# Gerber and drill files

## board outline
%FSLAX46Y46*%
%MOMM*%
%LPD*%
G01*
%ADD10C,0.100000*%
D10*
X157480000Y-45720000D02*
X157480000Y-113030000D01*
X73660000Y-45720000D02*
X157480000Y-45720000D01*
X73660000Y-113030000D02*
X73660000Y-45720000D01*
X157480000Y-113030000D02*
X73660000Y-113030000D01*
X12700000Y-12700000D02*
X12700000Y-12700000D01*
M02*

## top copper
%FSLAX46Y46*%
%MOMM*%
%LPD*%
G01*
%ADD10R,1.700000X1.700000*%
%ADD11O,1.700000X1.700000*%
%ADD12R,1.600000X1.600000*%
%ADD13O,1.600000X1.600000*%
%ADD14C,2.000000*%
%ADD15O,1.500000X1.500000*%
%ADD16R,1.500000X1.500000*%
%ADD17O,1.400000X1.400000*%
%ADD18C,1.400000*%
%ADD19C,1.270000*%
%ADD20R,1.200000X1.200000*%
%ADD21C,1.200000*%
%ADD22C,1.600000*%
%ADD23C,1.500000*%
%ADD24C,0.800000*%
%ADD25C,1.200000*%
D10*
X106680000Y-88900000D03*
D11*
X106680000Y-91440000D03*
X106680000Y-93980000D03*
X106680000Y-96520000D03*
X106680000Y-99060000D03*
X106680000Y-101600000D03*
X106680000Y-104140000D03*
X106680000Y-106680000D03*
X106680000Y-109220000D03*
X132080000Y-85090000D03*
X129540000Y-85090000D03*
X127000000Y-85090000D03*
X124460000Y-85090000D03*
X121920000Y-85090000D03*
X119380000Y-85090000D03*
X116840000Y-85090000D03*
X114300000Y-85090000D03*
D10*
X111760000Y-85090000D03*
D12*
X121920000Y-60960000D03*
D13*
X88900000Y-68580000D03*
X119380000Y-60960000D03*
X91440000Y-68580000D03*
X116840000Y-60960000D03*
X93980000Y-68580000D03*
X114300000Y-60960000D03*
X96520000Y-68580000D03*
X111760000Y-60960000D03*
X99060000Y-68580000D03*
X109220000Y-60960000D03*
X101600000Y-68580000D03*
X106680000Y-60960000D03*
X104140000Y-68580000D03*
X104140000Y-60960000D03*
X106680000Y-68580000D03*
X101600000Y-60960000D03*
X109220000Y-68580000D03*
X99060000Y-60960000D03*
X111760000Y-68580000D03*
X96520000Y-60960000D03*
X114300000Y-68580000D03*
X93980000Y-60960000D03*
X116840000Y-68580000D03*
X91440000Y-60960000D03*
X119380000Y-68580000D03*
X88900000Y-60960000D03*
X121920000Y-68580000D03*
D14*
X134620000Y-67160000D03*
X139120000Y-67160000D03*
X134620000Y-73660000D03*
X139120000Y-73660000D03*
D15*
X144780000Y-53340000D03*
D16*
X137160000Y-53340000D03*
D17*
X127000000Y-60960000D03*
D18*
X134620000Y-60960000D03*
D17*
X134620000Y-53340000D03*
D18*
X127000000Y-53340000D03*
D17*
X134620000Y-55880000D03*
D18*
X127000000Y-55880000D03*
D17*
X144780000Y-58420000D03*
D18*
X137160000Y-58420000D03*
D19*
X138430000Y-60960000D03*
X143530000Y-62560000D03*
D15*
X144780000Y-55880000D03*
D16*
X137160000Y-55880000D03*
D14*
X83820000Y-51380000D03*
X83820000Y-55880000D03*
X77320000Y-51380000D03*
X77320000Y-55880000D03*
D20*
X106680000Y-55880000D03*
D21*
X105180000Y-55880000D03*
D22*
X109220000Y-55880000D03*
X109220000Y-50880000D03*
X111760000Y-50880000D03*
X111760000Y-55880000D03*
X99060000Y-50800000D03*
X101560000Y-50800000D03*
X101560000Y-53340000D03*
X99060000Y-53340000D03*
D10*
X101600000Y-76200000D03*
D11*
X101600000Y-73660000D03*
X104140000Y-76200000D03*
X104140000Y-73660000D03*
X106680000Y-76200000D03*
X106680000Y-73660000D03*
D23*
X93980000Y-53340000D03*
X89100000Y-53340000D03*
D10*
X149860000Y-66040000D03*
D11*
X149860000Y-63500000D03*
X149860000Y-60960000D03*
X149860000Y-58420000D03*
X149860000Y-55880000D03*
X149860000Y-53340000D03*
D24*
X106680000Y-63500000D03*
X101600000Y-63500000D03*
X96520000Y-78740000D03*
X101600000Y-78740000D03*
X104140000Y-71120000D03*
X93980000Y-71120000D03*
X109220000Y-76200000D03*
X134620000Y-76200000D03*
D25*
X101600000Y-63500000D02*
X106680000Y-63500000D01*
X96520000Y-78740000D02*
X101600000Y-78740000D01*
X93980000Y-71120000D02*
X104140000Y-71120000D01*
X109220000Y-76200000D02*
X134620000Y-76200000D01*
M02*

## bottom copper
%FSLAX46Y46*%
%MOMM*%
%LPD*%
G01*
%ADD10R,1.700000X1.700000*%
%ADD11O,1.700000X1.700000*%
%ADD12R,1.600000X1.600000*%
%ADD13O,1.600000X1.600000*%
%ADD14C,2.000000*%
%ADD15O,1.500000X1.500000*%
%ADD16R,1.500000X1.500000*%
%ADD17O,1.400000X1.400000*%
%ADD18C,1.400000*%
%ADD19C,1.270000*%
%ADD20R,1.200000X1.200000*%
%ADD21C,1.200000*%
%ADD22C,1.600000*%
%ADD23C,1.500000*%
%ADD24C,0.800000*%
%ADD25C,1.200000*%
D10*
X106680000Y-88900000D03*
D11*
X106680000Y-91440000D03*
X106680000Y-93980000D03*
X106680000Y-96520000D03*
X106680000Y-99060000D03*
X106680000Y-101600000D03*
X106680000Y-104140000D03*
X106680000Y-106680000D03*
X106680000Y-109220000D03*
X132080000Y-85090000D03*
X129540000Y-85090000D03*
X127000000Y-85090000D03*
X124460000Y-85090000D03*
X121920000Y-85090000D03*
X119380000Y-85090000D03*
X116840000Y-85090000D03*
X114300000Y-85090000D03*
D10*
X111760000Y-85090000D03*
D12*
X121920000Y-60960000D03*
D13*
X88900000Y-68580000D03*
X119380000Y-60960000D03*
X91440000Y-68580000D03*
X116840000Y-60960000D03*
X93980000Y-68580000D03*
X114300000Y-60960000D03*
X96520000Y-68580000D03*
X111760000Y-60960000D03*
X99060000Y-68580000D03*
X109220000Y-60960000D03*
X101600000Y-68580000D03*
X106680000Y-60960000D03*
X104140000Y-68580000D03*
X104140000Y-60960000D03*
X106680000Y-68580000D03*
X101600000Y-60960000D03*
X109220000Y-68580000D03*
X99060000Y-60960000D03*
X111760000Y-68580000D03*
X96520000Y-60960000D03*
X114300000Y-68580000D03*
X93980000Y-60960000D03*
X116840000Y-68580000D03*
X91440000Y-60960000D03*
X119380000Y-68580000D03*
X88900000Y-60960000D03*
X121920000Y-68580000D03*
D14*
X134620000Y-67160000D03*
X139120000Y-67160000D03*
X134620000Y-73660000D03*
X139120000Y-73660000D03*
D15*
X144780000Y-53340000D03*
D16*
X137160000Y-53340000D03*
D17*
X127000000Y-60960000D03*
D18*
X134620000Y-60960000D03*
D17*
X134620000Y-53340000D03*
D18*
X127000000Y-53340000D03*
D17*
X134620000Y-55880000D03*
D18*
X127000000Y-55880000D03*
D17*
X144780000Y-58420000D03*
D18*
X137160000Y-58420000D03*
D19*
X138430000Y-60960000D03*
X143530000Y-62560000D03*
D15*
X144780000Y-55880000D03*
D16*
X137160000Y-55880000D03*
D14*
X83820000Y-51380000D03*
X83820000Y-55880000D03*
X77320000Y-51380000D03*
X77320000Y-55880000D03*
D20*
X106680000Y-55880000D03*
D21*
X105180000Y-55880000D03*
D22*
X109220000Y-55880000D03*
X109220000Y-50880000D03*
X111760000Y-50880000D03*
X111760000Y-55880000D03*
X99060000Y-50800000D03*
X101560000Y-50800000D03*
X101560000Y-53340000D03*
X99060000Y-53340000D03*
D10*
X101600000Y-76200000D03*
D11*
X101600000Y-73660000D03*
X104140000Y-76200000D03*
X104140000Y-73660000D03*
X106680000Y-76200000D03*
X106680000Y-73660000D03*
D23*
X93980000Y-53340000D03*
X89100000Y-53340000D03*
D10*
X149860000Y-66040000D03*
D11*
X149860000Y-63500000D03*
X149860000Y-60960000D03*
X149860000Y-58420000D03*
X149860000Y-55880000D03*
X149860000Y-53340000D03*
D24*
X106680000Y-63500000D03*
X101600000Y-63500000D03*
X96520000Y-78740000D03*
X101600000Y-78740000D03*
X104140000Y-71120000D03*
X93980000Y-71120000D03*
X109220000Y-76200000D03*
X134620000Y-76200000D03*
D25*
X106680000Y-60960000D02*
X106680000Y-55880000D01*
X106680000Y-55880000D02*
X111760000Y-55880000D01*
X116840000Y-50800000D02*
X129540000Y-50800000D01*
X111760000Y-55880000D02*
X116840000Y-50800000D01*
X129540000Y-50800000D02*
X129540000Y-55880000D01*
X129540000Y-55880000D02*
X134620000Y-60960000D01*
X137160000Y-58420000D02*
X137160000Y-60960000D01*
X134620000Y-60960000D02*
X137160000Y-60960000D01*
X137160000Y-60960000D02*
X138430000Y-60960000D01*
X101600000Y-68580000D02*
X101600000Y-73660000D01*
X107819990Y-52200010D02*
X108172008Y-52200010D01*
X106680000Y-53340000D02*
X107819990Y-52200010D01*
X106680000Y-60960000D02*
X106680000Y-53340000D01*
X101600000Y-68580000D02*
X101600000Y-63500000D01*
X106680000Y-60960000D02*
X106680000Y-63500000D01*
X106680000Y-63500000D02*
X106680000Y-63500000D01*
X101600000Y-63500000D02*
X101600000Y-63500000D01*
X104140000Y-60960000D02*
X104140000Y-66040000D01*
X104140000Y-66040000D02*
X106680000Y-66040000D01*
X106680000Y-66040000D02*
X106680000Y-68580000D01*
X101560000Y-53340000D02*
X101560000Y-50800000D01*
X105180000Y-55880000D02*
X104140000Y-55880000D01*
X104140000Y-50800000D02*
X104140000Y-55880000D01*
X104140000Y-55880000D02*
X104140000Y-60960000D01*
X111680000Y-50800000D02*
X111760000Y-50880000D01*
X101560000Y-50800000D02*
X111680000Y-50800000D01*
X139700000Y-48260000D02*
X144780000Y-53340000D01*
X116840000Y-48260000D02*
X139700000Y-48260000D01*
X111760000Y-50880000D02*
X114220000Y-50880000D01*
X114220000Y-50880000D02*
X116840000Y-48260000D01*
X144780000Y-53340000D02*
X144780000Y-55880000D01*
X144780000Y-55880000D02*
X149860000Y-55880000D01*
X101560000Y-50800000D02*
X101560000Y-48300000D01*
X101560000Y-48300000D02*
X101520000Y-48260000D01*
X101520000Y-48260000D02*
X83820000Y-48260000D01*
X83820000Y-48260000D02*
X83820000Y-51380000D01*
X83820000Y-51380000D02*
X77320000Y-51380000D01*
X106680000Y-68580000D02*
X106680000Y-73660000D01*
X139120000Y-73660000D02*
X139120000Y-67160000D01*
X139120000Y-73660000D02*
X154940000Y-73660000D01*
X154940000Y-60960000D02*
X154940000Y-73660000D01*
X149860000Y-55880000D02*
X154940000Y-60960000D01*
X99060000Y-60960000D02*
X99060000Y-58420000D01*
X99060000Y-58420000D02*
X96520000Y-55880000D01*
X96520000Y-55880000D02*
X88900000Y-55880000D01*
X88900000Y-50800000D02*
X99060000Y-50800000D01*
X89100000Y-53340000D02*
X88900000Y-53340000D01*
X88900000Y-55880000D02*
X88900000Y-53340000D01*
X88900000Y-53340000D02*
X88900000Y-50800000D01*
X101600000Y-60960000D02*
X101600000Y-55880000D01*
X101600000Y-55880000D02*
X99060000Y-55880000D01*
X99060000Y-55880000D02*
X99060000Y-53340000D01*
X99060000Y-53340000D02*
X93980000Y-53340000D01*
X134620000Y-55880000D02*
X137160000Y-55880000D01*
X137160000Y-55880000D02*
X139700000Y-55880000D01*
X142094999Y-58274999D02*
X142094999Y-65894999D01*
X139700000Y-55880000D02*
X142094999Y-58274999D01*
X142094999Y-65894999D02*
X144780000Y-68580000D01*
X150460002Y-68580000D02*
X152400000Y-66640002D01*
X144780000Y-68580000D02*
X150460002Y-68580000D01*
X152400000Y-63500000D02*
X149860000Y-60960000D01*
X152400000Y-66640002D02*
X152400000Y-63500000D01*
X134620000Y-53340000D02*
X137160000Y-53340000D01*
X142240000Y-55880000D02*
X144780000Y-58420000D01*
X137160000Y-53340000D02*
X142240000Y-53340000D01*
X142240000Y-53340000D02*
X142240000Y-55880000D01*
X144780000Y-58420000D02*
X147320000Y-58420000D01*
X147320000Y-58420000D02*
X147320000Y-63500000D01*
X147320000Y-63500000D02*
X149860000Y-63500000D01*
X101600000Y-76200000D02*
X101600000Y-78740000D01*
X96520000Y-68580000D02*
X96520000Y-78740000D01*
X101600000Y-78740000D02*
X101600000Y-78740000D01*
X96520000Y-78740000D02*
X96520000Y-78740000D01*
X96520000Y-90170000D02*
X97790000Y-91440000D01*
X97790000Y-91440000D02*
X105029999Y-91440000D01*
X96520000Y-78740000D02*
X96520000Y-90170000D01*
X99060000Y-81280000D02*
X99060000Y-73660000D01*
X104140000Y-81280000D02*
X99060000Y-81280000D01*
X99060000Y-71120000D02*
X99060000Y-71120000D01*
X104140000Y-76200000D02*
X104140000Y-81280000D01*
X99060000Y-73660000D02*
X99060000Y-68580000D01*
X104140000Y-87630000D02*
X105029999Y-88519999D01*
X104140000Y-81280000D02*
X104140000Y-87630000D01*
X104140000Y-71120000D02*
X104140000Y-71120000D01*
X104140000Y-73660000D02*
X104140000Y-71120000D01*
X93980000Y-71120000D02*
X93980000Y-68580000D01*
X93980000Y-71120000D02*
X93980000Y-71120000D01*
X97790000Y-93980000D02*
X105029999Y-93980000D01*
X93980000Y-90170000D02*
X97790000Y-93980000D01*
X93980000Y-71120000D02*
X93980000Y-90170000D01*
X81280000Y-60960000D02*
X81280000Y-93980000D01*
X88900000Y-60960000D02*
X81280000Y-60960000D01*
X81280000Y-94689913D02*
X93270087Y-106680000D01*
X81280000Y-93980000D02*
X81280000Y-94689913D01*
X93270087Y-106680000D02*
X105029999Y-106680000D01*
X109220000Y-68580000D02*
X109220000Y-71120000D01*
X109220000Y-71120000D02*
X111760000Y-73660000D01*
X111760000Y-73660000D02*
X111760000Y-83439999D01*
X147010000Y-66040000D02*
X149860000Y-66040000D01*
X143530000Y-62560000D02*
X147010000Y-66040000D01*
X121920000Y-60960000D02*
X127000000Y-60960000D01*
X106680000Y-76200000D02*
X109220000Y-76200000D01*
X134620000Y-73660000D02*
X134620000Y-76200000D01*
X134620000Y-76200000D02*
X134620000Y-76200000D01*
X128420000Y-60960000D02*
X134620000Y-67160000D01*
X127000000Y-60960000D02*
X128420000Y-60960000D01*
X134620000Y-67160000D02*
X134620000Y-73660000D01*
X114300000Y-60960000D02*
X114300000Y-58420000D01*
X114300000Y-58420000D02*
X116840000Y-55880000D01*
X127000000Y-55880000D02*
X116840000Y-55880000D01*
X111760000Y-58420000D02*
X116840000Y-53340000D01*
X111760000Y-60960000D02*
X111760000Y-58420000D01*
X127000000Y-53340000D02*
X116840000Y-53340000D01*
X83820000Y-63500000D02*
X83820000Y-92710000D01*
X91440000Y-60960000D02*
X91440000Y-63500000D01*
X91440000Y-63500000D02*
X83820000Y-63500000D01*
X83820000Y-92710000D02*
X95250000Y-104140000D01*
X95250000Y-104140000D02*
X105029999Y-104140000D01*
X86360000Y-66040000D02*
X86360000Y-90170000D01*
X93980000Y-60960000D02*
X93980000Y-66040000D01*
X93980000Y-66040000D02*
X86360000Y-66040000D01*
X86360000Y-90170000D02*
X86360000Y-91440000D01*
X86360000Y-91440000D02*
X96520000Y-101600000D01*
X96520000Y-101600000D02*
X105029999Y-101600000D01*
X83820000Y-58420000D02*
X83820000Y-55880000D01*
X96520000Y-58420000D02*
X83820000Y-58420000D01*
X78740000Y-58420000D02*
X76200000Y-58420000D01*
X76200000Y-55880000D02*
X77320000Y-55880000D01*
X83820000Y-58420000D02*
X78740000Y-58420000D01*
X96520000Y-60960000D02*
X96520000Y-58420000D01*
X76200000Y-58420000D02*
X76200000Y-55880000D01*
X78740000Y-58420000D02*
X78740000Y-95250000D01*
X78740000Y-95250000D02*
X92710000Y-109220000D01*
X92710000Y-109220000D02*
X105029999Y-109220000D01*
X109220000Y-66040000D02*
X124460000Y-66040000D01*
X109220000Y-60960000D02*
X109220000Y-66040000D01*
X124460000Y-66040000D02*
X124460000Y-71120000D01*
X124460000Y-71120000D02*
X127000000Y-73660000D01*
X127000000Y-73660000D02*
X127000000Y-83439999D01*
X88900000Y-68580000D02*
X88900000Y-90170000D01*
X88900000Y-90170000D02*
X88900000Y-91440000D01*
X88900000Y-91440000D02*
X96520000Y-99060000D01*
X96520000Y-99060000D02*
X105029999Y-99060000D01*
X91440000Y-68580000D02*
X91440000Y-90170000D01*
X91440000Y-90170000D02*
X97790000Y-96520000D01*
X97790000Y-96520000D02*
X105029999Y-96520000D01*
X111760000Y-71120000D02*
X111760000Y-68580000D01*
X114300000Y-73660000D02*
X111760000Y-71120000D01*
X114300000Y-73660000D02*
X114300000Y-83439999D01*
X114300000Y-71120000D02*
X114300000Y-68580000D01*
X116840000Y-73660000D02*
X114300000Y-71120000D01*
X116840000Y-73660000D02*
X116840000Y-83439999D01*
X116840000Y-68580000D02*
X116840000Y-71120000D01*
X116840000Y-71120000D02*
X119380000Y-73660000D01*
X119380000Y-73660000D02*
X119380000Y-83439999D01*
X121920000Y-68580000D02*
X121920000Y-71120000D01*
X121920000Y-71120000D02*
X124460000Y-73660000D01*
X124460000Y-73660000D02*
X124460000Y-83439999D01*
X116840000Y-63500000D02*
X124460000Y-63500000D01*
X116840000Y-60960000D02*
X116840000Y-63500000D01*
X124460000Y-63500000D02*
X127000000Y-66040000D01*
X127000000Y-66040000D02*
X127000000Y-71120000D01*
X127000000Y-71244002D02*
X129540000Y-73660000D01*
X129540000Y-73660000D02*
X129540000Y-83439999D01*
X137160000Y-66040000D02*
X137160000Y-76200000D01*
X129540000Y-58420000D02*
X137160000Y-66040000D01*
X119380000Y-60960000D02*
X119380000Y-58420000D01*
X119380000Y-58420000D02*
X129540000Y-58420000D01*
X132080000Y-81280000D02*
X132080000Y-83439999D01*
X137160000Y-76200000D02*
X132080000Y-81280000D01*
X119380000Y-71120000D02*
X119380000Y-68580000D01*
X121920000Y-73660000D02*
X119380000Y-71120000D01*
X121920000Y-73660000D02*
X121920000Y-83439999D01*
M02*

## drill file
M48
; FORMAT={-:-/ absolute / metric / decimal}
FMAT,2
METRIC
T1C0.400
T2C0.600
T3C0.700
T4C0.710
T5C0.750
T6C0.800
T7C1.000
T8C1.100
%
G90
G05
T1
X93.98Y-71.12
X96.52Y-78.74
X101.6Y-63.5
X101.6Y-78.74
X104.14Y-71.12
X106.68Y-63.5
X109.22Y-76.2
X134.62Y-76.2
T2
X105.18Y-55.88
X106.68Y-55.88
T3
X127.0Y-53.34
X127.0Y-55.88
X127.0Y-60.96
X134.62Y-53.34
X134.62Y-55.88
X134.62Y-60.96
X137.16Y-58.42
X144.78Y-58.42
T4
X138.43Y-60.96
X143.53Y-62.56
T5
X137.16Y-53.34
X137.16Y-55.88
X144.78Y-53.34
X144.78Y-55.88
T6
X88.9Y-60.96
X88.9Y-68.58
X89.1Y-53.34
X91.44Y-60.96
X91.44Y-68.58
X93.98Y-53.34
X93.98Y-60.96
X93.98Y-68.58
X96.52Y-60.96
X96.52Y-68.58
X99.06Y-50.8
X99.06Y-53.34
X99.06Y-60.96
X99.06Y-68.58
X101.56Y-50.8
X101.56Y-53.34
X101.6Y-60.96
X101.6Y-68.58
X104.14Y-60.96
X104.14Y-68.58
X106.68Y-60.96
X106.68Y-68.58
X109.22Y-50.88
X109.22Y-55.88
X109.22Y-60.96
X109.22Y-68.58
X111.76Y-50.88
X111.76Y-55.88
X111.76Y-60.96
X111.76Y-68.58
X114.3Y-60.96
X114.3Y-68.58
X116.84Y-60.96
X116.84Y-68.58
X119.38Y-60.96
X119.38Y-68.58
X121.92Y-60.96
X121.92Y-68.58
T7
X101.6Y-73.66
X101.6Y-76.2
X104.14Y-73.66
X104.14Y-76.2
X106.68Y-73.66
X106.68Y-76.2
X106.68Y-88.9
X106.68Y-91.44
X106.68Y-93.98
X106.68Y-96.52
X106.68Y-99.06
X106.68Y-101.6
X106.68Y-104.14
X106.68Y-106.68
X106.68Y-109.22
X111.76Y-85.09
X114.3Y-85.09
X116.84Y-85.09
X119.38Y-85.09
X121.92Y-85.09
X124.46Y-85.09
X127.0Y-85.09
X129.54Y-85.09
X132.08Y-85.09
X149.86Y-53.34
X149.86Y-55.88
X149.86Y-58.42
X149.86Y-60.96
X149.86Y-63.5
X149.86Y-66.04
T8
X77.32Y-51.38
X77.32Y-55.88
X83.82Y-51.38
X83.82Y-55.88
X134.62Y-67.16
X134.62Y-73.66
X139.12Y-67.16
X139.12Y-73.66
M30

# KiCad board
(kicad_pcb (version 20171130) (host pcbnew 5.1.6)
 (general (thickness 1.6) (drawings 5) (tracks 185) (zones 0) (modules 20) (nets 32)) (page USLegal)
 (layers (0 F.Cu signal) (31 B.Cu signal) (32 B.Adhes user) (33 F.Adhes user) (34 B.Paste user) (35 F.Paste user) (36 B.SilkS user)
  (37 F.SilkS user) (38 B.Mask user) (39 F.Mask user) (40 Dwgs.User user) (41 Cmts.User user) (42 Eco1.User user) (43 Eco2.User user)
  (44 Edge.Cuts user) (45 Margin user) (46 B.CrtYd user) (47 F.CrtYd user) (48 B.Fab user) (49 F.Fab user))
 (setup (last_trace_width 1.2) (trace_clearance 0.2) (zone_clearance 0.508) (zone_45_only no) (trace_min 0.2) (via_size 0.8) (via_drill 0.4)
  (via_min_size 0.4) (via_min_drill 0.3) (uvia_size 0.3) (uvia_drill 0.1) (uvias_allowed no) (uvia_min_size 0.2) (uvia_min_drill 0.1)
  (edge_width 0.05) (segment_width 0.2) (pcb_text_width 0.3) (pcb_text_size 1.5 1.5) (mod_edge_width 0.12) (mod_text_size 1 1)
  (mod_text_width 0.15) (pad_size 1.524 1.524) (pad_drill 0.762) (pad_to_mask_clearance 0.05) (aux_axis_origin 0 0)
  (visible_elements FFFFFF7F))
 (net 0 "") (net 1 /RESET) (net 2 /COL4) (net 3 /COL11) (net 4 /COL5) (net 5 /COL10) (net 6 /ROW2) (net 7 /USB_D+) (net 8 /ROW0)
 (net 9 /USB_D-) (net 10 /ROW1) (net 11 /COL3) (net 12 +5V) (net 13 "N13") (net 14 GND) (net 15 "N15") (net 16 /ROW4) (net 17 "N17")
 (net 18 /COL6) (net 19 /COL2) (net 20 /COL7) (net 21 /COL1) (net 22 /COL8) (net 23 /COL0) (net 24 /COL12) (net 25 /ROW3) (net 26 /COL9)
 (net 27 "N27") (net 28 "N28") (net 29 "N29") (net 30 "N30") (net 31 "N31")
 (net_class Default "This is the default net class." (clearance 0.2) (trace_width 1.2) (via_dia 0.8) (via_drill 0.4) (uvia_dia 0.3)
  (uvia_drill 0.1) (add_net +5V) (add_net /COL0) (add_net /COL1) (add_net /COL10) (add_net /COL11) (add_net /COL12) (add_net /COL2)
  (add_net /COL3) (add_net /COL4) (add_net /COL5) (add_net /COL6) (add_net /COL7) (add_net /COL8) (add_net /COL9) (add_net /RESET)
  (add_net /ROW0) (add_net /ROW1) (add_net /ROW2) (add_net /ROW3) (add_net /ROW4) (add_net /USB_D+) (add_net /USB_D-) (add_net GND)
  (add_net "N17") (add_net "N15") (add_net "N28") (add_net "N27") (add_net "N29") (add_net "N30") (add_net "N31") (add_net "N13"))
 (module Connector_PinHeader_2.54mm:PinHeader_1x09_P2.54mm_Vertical (layer F.Cu) (at 106.68 88.9)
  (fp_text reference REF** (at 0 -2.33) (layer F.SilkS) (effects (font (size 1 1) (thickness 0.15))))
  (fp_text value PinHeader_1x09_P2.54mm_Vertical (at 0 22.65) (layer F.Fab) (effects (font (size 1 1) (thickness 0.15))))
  (pad 1 thru_hole rect (at 0 0) (size 1.7 1.7) (drill 1) (layers *.Cu *.Mask))
  (pad 2 thru_hole oval (at 0 2.54) (size 1.7 1.7) (drill 1) (layers *.Cu *.Mask))
  (pad 3 thru_hole oval (at 0 5.08) (size 1.7 1.7) (drill 1) (layers *.Cu *.Mask))
  (pad 4 thru_hole oval (at 0 7.62) (size 1.7 1.7) (drill 1) (layers *.Cu *.Mask))
  (pad 5 thru_hole oval (at 0 10.16) (size 1.7 1.7) (drill 1) (layers *.Cu *.Mask))
  (pad 6 thru_hole oval (at 0 12.7) (size 1.7 1.7) (drill 1) (layers *.Cu *.Mask))
  (pad 7 thru_hole oval (at 0 15.24) (size 1.7 1.7) (drill 1) (layers *.Cu *.Mask))
  (pad 8 thru_hole oval (at 0 17.78) (size 1.7 1.7) (drill 1) (layers *.Cu *.Mask))
  (pad 9 thru_hole oval (at 0 20.32) (size 1.7 1.7) (drill 1) (layers *.Cu *.Mask)))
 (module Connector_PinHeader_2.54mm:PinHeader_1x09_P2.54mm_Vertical (layer F.Cu) (at 111.76 85.09 90)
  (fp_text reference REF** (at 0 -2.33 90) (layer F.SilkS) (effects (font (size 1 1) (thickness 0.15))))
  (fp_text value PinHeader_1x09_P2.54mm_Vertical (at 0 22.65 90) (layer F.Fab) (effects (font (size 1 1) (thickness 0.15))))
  (pad 9 thru_hole oval (at 0 20.32 90) (size 1.7 1.7) (drill 1) (layers *.Cu *.Mask))
  (pad 8 thru_hole oval (at 0 17.78 90) (size 1.7 1.7) (drill 1) (layers *.Cu *.Mask))
  (pad 7 thru_hole oval (at 0 15.24 90) (size 1.7 1.7) (drill 1) (layers *.Cu *.Mask))
  (pad 6 thru_hole oval (at 0 12.7 90) (size 1.7 1.7) (drill 1) (layers *.Cu *.Mask))
  (pad 5 thru_hole oval (at 0 10.16 90) (size 1.7 1.7) (drill 1) (layers *.Cu *.Mask))
  (pad 4 thru_hole oval (at 0 7.62 90) (size 1.7 1.7) (drill 1) (layers *.Cu *.Mask))
  (pad 3 thru_hole oval (at 0 5.08 90) (size 1.7 1.7) (drill 1) (layers *.Cu *.Mask))
  (pad 2 thru_hole oval (at 0 2.54 90) (size 1.7 1.7) (drill 1) (layers *.Cu *.Mask))
  (pad 1 thru_hole rect (at 0 0 90) (size 1.7 1.7) (drill 1) (layers *.Cu *.Mask)))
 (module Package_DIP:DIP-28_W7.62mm (layer F.Cu) (at 121.92 60.96 270)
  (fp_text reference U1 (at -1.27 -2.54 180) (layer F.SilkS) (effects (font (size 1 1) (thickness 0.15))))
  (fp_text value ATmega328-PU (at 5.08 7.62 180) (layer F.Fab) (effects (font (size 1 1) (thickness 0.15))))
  (pad 1 thru_hole rect (at 0 0 270) (size 1.6 1.6) (drill 0.8) (layers *.Cu *.Mask) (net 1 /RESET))
  (pad 15 thru_hole oval (at 7.62 33.02 270) (size 1.6 1.6) (drill 0.8) (layers *.Cu *.Mask) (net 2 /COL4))
  (pad 2 thru_hole oval (at 0 2.54 270) (size 1.6 1.6) (drill 0.8) (layers *.Cu *.Mask) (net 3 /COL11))
  (pad 16 thru_hole oval (at 7.62 30.48 270) (size 1.6 1.6) (drill 0.8) (layers *.Cu *.Mask) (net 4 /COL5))
  (pad 3 thru_hole oval (at 0 5.08 270) (size 1.6 1.6) (drill 0.8) (layers *.Cu *.Mask) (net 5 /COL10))
  (pad 17 thru_hole oval (at 7.62 27.94 270) (size 1.6 1.6) (drill 0.8) (layers *.Cu *.Mask) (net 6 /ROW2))
  (pad 4 thru_hole oval (at 0 7.62 270) (size 1.6 1.6) (drill 0.8) (layers *.Cu *.Mask) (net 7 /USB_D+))
  (pad 18 thru_hole oval (at 7.62 25.4 270) (size 1.6 1.6) (drill 0.8) (layers *.Cu *.Mask) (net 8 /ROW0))
  (pad 5 thru_hole oval (at 0 10.16 270) (size 1.6 1.6) (drill 0.8) (layers *.Cu *.Mask) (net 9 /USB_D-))
  (pad 19 thru_hole oval (at 7.62 22.86 270) (size 1.6 1.6) (drill 0.8) (layers *.Cu *.Mask) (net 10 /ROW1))
  (pad 6 thru_hole oval (at 0 12.7 270) (size 1.6 1.6) (drill 0.8) (layers *.Cu *.Mask) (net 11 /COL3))
  (pad 20 thru_hole oval (at 7.62 20.32 270) (size 1.6 1.6) (drill 0.8) (layers *.Cu *.Mask) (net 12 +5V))
  (pad 7 thru_hole oval (at 0 15.24 270) (size 1.6 1.6) (drill 0.8) (layers *.Cu *.Mask) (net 12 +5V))
  (pad 21 thru_hole oval (at 7.62 17.78 270) (size 1.6 1.6) (drill 0.8) (layers *.Cu *.Mask) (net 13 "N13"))
  (pad 8 thru_hole oval (at 0 17.78 270) (size 1.6 1.6) (drill 0.8) (layers *.Cu *.Mask) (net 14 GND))
  (pad 22 thru_hole oval (at 7.62 15.24 270) (size 1.6 1.6) (drill 0.8) (layers *.Cu *.Mask) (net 14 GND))
  (pad 9 thru_hole oval (at 0 20.32 270) (size 1.6 1.6) (drill 0.8) (layers *.Cu *.Mask) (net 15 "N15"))
  (pad 23 thru_hole oval (at 7.62 12.7 270) (size 1.6 1.6) (drill 0.8) (layers *.Cu *.Mask) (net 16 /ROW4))
  (pad 10 thru_hole oval (at 0 22.86 270) (size 1.6 1.6) (drill 0.8) (layers *.Cu *.Mask) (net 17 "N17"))
  (pad 24 thru_hole oval (at 7.62 10.16 270) (size 1.6 1.6) (drill 0.8) (layers *.Cu *.Mask) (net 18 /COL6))
  (pad 11 thru_hole oval (at 0 25.4 270) (size 1.6 1.6) (drill 0.8) (layers *.Cu *.Mask) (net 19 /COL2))
  (pad 25 thru_hole oval (at 7.62 7.62 270) (size 1.6 1.6) (drill 0.8) (layers *.Cu *.Mask) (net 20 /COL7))
  (pad 12 thru_hole oval (at 0 27.94 270) (size 1.6 1.6) (drill 0.8) (layers *.Cu *.Mask) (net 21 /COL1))
  (pad 26 thru_hole oval (at 7.62 5.08 270) (size 1.6 1.6) (drill 0.8) (layers *.Cu *.Mask) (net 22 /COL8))
  (pad 13 thru_hole oval (at 0 30.48 270) (size 1.6 1.6) (drill 0.8) (layers *.Cu *.Mask) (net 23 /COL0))
  (pad 27 thru_hole oval (at 7.62 2.54 270) (size 1.6 1.6) (drill 0.8) (layers *.Cu *.Mask) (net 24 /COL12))
  (pad 14 thru_hole oval (at 0 33.02 270) (size 1.6 1.6) (drill 0.8) (layers *.Cu *.Mask) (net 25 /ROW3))
  (pad 28 thru_hole oval (at 7.62 0 270) (size 1.6 1.6) (drill 0.8) (layers *.Cu *.Mask) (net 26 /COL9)))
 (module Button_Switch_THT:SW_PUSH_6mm (layer F.Cu) (at 134.62 73.66 90)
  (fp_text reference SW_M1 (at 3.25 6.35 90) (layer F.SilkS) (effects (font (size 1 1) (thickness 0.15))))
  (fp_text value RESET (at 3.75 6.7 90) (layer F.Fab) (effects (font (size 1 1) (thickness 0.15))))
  (pad 1 thru_hole circle (at 6.5 0 180) (size 2 2) (drill 1.1) (layers *.Cu *.Mask) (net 1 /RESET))
  (pad 2 thru_hole circle (at 6.5 4.5 180) (size 2 2) (drill 1.1) (layers *.Cu *.Mask) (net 14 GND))
  (pad 1 thru_hole circle (at 0 0 180) (size 2 2) (drill 1.1) (layers *.Cu *.Mask) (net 1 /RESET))
  (pad 2 thru_hole circle (at 0 4.5 180) (size 2 2) (drill 1.1) (layers *.Cu *.Mask) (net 14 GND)))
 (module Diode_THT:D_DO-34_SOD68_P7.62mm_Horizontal (layer F.Cu) (at 137.16 53.34)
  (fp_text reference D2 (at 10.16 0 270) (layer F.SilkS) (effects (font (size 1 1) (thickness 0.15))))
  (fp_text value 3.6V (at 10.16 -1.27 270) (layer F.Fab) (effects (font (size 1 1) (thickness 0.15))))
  (pad 2 thru_hole oval (at 7.62 0) (size 1.5 1.5) (drill 0.75) (layers *.Cu *.Mask) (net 14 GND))
  (pad 1 thru_hole rect (at 0 0) (size 1.5 1.5) (drill 0.75) (layers *.Cu *.Mask) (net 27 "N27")))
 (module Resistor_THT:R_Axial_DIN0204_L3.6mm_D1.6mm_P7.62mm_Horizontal (layer F.Cu) (at 134.62 60.96 180)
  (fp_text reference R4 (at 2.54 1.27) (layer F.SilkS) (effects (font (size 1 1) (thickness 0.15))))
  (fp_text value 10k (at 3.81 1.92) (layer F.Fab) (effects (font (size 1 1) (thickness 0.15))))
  (pad 2 thru_hole oval (at 7.62 0 180) (size 1.4 1.4) (drill 0.7) (layers *.Cu *.Mask) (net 1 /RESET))
  (pad 1 thru_hole circle (at 0 0 180) (size 1.4 1.4) (drill 0.7) (layers *.Cu *.Mask) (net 12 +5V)))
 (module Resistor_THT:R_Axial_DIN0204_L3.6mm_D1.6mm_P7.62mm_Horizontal (layer F.Cu) (at 127 53.34)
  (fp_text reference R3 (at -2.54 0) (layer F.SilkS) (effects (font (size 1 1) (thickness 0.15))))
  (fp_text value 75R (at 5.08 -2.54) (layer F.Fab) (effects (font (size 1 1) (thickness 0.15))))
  (pad 2 thru_hole oval (at 7.62 0) (size 1.4 1.4) (drill 0.7) (layers *.Cu *.Mask) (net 27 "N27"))
  (pad 1 thru_hole circle (at 0 0) (size 1.4 1.4) (drill 0.7) (layers *.Cu *.Mask) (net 9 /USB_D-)))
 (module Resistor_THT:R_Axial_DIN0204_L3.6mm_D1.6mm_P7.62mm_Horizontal (layer F.Cu) (at 127 55.88)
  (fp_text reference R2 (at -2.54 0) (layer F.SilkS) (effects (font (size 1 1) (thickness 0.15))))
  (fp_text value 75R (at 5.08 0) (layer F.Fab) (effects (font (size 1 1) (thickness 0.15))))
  (pad 2 thru_hole oval (at 7.62 0) (size 1.4 1.4) (drill 0.7) (layers *.Cu *.Mask) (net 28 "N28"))
  (pad 1 thru_hole circle (at 0 0) (size 1.4 1.4) (drill 0.7) (layers *.Cu *.Mask) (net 7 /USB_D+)))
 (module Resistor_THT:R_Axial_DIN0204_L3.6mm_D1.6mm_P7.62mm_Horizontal (layer F.Cu) (at 137.16 58.42)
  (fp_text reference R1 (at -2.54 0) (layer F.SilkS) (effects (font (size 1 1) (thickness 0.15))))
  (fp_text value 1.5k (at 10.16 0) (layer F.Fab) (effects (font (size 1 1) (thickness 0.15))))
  (pad 2 thru_hole oval (at 7.62 0) (size 1.4 1.4) (drill 0.7) (layers *.Cu *.Mask) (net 27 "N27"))
  (pad 1 thru_hole circle (at 0 0) (size 1.4 1.4) (drill 0.7) (layers *.Cu *.Mask) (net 12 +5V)))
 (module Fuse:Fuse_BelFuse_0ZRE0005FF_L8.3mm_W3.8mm (layer F.Cu) (at 138.43 60.96)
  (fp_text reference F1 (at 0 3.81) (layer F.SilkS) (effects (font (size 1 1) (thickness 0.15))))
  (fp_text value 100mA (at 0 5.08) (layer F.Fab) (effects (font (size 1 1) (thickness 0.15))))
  (pad 1 thru_hole circle (at 0 0) (size 1.27 1.27) (drill 0.71) (layers *.Cu *.Mask) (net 12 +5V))
  (pad 2 thru_hole circle (at 5.1 1.6) (size 1.27 1.27) (drill 0.71) (layers *.Cu *.Mask) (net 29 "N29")))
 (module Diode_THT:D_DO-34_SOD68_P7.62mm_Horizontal (layer F.Cu) (at 137.16 55.88)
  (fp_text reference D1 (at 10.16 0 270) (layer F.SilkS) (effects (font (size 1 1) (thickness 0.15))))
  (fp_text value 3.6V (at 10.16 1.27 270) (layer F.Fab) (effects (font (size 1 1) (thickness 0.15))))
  (pad 2 thru_hole oval (at 7.62 0) (size 1.5 1.5) (drill 0.75) (layers *.Cu *.Mask) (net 14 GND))
  (pad 1 thru_hole rect (at 0 0) (size 1.5 1.5) (drill 0.75) (layers *.Cu *.Mask) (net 28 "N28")))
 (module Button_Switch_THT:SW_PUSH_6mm (layer F.Cu) (at 83.82 55.88 180)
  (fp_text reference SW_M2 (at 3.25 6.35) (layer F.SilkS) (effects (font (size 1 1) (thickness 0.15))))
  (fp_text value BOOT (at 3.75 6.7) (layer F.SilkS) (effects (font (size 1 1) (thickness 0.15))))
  (pad 2 thru_hole circle (at 0 4.5 270) (size 2 2) (drill 1.1) (layers *.Cu *.Mask) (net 14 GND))
  (pad 1 thru_hole circle (at 0 0 270) (size 2 2) (drill 1.1) (layers *.Cu *.Mask) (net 19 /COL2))
  (pad 2 thru_hole circle (at 6.5 4.5 270) (size 2 2) (drill 1.1) (layers *.Cu *.Mask) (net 14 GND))
  (pad 1 thru_hole circle (at 6.5 0 270) (size 2 2) (drill 1.1) (layers *.Cu *.Mask) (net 19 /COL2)))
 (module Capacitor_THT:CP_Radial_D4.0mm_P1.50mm (layer F.Cu) (at 106.68 55.88 180)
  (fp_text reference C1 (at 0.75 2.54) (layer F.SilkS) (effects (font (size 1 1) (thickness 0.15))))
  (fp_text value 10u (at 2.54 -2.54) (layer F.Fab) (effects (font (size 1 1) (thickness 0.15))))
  (pad 1 thru_hole rect (at 0 0 180) (size 1.2 1.2) (drill 0.6) (layers *.Cu *.Mask) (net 12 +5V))
  (pad 2 thru_hole circle (at 1.5 0 180) (size 1.2 1.2) (drill 0.6) (layers *.Cu *.Mask) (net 14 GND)))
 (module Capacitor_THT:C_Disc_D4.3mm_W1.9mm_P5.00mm (layer F.Cu) (at 109.22 55.88 90)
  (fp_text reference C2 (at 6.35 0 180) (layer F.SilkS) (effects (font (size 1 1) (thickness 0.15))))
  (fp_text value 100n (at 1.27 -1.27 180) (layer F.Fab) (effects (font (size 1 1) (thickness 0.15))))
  (pad 1 thru_hole circle (at 0 0 90) (size 1.6 1.6) (drill 0.8) (layers *.Cu *.Mask) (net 12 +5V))
  (pad 2 thru_hole circle (at 5 0 90) (size 1.6 1.6) (drill 0.8) (layers *.Cu *.Mask) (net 14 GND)))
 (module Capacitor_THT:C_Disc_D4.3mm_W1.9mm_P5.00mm (layer F.Cu) (at 111.76 55.88 90)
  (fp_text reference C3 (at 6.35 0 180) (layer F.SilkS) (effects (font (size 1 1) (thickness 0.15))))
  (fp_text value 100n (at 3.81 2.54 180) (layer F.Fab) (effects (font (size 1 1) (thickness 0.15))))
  (pad 2 thru_hole circle (at 5 0 90) (size 1.6 1.6) (drill 0.8) (layers *.Cu *.Mask) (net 14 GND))
  (pad 1 thru_hole circle (at 0 0 90) (size 1.6 1.6) (drill 0.8) (layers *.Cu *.Mask) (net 12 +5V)))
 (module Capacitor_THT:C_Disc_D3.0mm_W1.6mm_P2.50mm (layer F.Cu) (at 99.06 50.8)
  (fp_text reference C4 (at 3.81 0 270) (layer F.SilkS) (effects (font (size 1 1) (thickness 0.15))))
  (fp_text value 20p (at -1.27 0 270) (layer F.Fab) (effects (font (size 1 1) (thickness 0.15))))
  (pad 1 thru_hole circle (at 0 0) (size 1.6 1.6) (drill 0.8) (layers *.Cu *.Mask) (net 17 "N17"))
  (pad 2 thru_hole circle (at 2.5 0) (size 1.6 1.6) (drill 0.8) (layers *.Cu *.Mask) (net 14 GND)))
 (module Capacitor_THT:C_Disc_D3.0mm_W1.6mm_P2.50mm (layer F.Cu) (at 99.06 53.34)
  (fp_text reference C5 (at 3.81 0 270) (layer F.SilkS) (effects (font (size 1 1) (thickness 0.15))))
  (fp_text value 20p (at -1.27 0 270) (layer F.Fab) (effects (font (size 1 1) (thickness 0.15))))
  (pad 2 thru_hole circle (at 2.5 0) (size 1.6 1.6) (drill 0.8) (layers *.Cu *.Mask) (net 14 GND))
  (pad 1 thru_hole circle (at 0 0) (size 1.6 1.6) (drill 0.8) (layers *.Cu *.Mask) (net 15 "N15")))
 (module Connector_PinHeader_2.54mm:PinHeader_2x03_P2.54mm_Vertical (layer F.Cu) (at 101.6 76.2 90)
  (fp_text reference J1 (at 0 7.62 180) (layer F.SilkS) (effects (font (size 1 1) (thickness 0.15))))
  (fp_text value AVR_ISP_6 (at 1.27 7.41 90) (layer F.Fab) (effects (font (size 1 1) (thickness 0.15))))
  (pad 1 thru_hole rect (at 0 0 90) (size 1.7 1.7) (drill 1) (layers *.Cu *.Mask) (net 8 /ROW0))
  (pad 2 thru_hole oval (at 2.54 0 90) (size 1.7 1.7) (drill 1) (layers *.Cu *.Mask) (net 12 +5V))
  (pad 3 thru_hole oval (at 0 2.54 90) (size 1.7 1.7) (drill 1) (layers *.Cu *.Mask) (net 10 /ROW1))
  (pad 4 thru_hole oval (at 2.54 2.54 90) (size 1.7 1.7) (drill 1) (layers *.Cu *.Mask) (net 6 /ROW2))
  (pad 5 thru_hole oval (at 0 5.08 90) (size 1.7 1.7) (drill 1) (layers *.Cu *.Mask) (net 1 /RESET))
  (pad 6 thru_hole oval (at 2.54 5.08 90) (size 1.7 1.7) (drill 1) (layers *.Cu *.Mask) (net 14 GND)))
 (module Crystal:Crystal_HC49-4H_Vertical (layer F.Cu) (at 93.98 53.34 180)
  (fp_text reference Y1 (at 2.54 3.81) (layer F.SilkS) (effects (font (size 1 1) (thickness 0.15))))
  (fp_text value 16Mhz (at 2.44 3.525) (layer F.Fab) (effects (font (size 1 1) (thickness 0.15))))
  (pad 1 thru_hole circle (at 0 0 180) (size 1.5 1.5) (drill 0.8) (layers *.Cu *.Mask) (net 15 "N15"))
  (pad 2 thru_hole circle (at 4.88 0 180) (size 1.5 1.5) (drill 0.8) (layers *.Cu *.Mask) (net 17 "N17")))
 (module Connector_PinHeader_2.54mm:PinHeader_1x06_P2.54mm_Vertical (layer F.Cu) (at 149.86 66.04 180)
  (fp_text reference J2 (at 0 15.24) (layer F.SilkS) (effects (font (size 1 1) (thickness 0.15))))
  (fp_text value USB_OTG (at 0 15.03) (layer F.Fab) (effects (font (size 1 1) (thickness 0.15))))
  (pad 1 thru_hole rect (at 0 0 180) (size 1.7 1.7) (drill 1) (layers *.Cu *.Mask) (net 29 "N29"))
  (pad 2 thru_hole oval (at 0 2.54 180) (size 1.7 1.7) (drill 1) (layers *.Cu *.Mask) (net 27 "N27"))
  (pad 3 thru_hole oval (at 0 5.08 180) (size 1.7 1.7) (drill 1) (layers *.Cu *.Mask) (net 28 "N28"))
  (pad 4 thru_hole oval (at 0 7.62 180) (size 1.7 1.7) (drill 1) (layers *.Cu *.Mask) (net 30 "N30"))
  (pad 5 thru_hole oval (at 0 10.16 180) (size 1.7 1.7) (drill 1) (layers *.Cu *.Mask) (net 14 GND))
  (pad 6 thru_hole oval (at 0 12.7 180) (size 1.7 1.7) (drill 1) (layers *.Cu *.Mask) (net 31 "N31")))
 (gr_line (start 157.48 45.72) (end 157.48 113.03) (layer Edge.Cuts) (width 0.1))
 (gr_line (start 73.66 45.72) (end 157.48 45.72) (layer Edge.Cuts) (width 0.1))
 (gr_line (start 73.66 113.03) (end 73.66 45.72) (layer Edge.Cuts) (width 0.1))
 (gr_line (start 157.48 113.03) (end 73.66 113.03) (layer Edge.Cuts) (width 0.1))
 (gr_line (start 12.7 12.7) (end 12.7 12.7) (layer Edge.Cuts) (width 0.1))
 (segment (start 106.68 60.96) (end 106.68 55.88) (width 1.2) (layer B.Cu) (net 12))
 (segment (start 106.68 55.88) (end 111.76 55.88) (width 1.2) (layer B.Cu) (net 12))
 (segment (start 116.84 50.8) (end 129.54 50.8) (width 1.2) (layer B.Cu) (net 12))
 (segment (start 111.76 55.88) (end 116.84 50.8) (width 1.2) (layer B.Cu) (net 12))
 (segment (start 129.54 50.8) (end 129.54 55.88) (width 1.2) (layer B.Cu) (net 12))
 (segment (start 129.54 55.88) (end 134.62 60.96) (width 1.2) (layer B.Cu) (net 12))
 (segment (start 137.16 58.42) (end 137.16 60.96) (width 1.2) (layer B.Cu) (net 12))
 (segment (start 134.62 60.96) (end 137.16 60.96) (width 1.2) (layer B.Cu) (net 12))
 (segment (start 137.16 60.96) (end 138.43 60.96) (width 1.2) (layer B.Cu) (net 12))
 (segment (start 101.6 68.58) (end 101.6 73.66) (width 1.2) (layer B.Cu) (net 12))
 (segment (start 107.81999 52.20001) (end 108.172008 52.20001) (width 1.2) (layer B.Cu) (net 12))
 (segment (start 106.68 53.34) (end 107.81999 52.20001) (width 1.2) (layer B.Cu) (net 12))
 (segment (start 106.68 60.96) (end 106.68 53.34) (width 1.2) (layer B.Cu) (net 12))
 (segment (start 101.6 68.58) (end 101.6 63.5) (width 1.2) (layer B.Cu) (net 12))
 (segment (start 106.68 60.96) (end 106.68 63.5) (width 1.2) (layer B.Cu) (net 12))
 (segment (start 106.68 63.5) (end 106.68 63.5) (width 1.2) (layer B.Cu) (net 12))
 (via (at 106.68 63.5) (size 0.8) (drill 0.4) (layers F.Cu B.Cu) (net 12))
 (segment (start 101.6 63.5) (end 101.6 63.5) (width 1.2) (layer B.Cu) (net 12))
 (via (at 101.6 63.5) (size 0.8) (drill 0.4) (layers F.Cu B.Cu) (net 12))
 (segment (start 101.6 63.5) (end 106.68 63.5) (width 1.2) (layer F.Cu) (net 12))
 (segment (start 104.14 60.96) (end 104.14 66.04) (width 1.2) (layer B.Cu) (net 14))
 (segment (start 104.14 66.04) (end 106.68 66.04) (width 1.2) (layer B.Cu) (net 14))
 (segment (start 106.68 66.04) (end 106.68 68.58) (width 1.2) (layer B.Cu) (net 14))
 (segment (start 101.56 53.34) (end 101.56 50.8) (width 1.2) (layer B.Cu) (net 14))
 (segment (start 105.18 55.88) (end 104.14 55.88) (width 1.2) (layer B.Cu) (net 14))
 (segment (start 104.14 50.8) (end 104.14 55.88) (width 1.2) (layer B.Cu) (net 14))
 (segment (start 104.14 55.88) (end 104.14 60.96) (width 1.2) (layer B.Cu) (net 14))
 (segment (start 111.68 50.8) (end 111.76 50.88) (width 1.2) (layer B.Cu) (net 14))
 (segment (start 101.56 50.8) (end 111.68 50.8) (width 1.2) (layer B.Cu) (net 14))
 (segment (start 139.7 48.26) (end 144.78 53.34) (width 1.2) (layer B.Cu) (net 14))
 (segment (start 116.84 48.26) (end 139.7 48.26) (width 1.2) (layer B.Cu) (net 14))
 (segment (start 111.76 50.88) (end 114.22 50.88) (width 1.2) (layer B.Cu) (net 14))
 (segment (start 114.22 50.88) (end 116.84 48.26) (width 1.2) (layer B.Cu) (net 14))
 (segment (start 144.78 53.34) (end 144.78 55.88) (width 1.2) (layer B.Cu) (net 14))
 (segment (start 144.78 55.88) (end 149.86 55.88) (width 1.2) (layer B.Cu) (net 14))
 (segment (start 101.56 50.8) (end 101.56 48.3) (width 1.2) (layer B.Cu) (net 14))
 (segment (start 101.56 48.3) (end 101.52 48.26) (width 1.2) (layer B.Cu) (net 14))
 (segment (start 101.52 48.26) (end 83.82 48.26) (width 1.2) (layer B.Cu) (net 14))
 (segment (start 83.82 48.26) (end 83.82 51.38) (width 1.2) (layer B.Cu) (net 14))
 (segment (start 83.82 51.38) (end 77.32 51.38) (width 1.2) (layer B.Cu) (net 14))
 (segment (start 106.68 68.58) (end 106.68 73.66) (width 1.2) (layer B.Cu) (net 14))
 (segment (start 139.12 73.66) (end 139.12 67.16) (width 1.2) (layer B.Cu) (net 14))
 (segment (start 139.12 73.66) (end 154.94 73.66) (width 1.2) (layer B.Cu) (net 14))
 (segment (start 154.94 60.96) (end 154.94 73.66) (width 1.2) (layer B.Cu) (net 14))
 (segment (start 149.86 55.88) (end 154.94 60.96) (width 1.2) (layer B.Cu) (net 14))
 (segment (start 99.06 60.96) (end 99.06 58.42) (width 1.2) (layer B.Cu) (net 17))
 (segment (start 99.06 58.42) (end 96.52 55.88) (width 1.2) (layer B.Cu) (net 17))
 (segment (start 96.52 55.88) (end 88.9 55.88) (width 1.2) (layer B.Cu) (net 17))
 (segment (start 88.9 50.8) (end 99.06 50.8) (width 1.2) (layer B.Cu) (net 17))
 (segment (start 89.1 53.34) (end 88.9 53.34) (width 1.2) (layer B.Cu) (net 17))
 (segment (start 88.9 55.88) (end 88.9 53.34) (width 1.2) (layer B.Cu) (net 17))
 (segment (start 88.9 53.34) (end 88.9 50.8) (width 1.2) (layer B.Cu) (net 17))
 (segment (start 101.6 60.96) (end 101.6 55.88) (width 1.2) (layer B.Cu) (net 15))
 (segment (start 101.6 55.88) (end 99.06 55.88) (width 1.2) (layer B.Cu) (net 15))
 (segment (start 99.06 55.88) (end 99.06 53.34) (width 1.2) (layer B.Cu) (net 15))
 (segment (start 99.06 53.34) (end 93.98 53.34) (width 1.2) (layer B.Cu) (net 15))
 (segment (start 134.62 55.88) (end 137.16 55.88) (width 1.2) (layer B.Cu) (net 28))
 (segment (start 137.16 55.88) (end 139.7 55.88) (width 1.2) (layer B.Cu) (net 28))
 (segment (start 142.094999 58.274999) (end 142.094999 65.894999) (width 1.2) (layer B.Cu) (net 28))
 (segment (start 139.7 55.88) (end 142.094999 58.274999) (width 1.2) (layer B.Cu) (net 28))
 (segment (start 142.094999 65.894999) (end 144.78 68.58) (width 1.2) (layer B.Cu) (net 28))
 (segment (start 150.460002 68.58) (end 152.4 66.640002) (width 1.2) (layer B.Cu) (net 28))
 (segment (start 144.78 68.58) (end 150.460002 68.58) (width 1.2) (layer B.Cu) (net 28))
 (segment (start 152.4 63.5) (end 149.86 60.96) (width 1.2) (layer B.Cu) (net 28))
 (segment (start 152.4 66.640002) (end 152.4 63.5) (width 1.2) (layer B.Cu) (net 28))
 (segment (start 134.62 53.34) (end 137.16 53.34) (width 1.2) (layer B.Cu) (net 27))
 (segment (start 142.24 55.88) (end 144.78 58.42) (width 1.2) (layer B.Cu) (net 27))
 (segment (start 137.16 53.34) (end 142.24 53.34) (width 1.2) (layer B.Cu) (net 27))
 (segment (start 142.24 53.34) (end 142.24 55.88) (width 1.2) (layer B.Cu) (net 27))
 (segment (start 144.78 58.42) (end 147.32 58.42) (width 1.2) (layer B.Cu) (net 27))
 (segment (start 147.32 58.42) (end 147.32 63.5) (width 1.2) (layer B.Cu) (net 27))
 (segment (start 147.32 63.5) (end 149.86 63.5) (width 1.2) (layer B.Cu) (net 27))
 (segment (start 101.6 76.2) (end 101.6 78.74) (width 1.2) (layer B.Cu) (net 8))
 (segment (start 96.52 68.58) (end 96.52 78.74) (width 1.2) (layer B.Cu) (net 8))
 (segment (start 101.6 78.74) (end 101.6 78.74) (width 1.2) (layer B.Cu) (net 8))
 (segment (start 96.52 78.74) (end 101.6 78.74) (width 1.2) (layer F.Cu) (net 8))
 (via (at 96.52 78.74) (size 0.8) (drill 0.4) (layers F.Cu B.Cu) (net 8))
 (segment (start 96.52 78.74) (end 96.52 78.74) (width 1.2) (layer B.Cu) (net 8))
 (via (at 101.6 78.74) (size 0.8) (drill 0.4) (layers F.Cu B.Cu) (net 8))
 (segment (start 96.52 90.17) (end 97.79 91.44) (width 1.2) (layer B.Cu) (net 8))
 (segment (start 97.79 91.44) (end 105.029999 91.44) (width 1.2) (layer B.Cu) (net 8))
 (segment (start 96.52 78.74) (end 96.52 90.17) (width 1.2) (layer B.Cu) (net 8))
 (segment (start 99.06 81.28) (end 99.06 73.66) (width 1.2) (layer B.Cu) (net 10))
 (segment (start 104.14 81.28) (end 99.06 81.28) (width 1.2) (layer B.Cu) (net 10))
 (segment (start 99.06 71.12) (end 99.06 71.12) (width 1.2) (layer B.Cu) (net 10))
 (segment (start 104.14 76.2) (end 104.14 81.28) (width 1.2) (layer B.Cu) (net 10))
 (segment (start 99.06 73.66) (end 99.06 68.58) (width 1.2) (layer B.Cu) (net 10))
 (segment (start 104.14 87.63) (end 105.029999 88.519999) (width 1.2) (layer B.Cu) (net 10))
 (segment (start 104.14 81.28) (end 104.14 87.63) (width 1.2) (layer B.Cu) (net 10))
 (segment (start 104.14 71.12) (end 104.14 71.12) (width 1.2) (layer B.Cu) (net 6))
 (via (at 104.14 71.12) (size 0.8) (drill 0.4) (layers F.Cu B.Cu) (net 6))
 (segment (start 104.14 73.66) (end 104.14 71.12) (width 1.2) (layer B.Cu) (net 6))
 (segment (start 93.98 71.12) (end 93.98 68.58) (width 1.2) (layer B.Cu) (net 6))
 (segment (start 93.98 71.12) (end 104.14 71.12) (width 1.2) (layer F.Cu) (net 6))
 (via (at 93.98 71.12) (size 0.8) (drill 0.4) (layers F.Cu B.Cu) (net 6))
 (segment (start 93.98 71.12) (end 93.98 71.12) (width 1.2) (layer B.Cu) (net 6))
 (segment (start 97.79 93.98) (end 105.029999 93.98) (width 1.2) (layer B.Cu) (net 6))
 (segment (start 93.98 90.17) (end 97.79 93.98) (width 1.2) (layer B.Cu) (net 6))
 (segment (start 93.98 71.12) (end 93.98 90.17) (width 1.2) (layer B.Cu) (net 6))
 (segment (start 81.28 60.96) (end 81.28 93.98) (width 1.2) (layer B.Cu) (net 25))
 (segment (start 88.9 60.96) (end 81.28 60.96) (width 1.2) (layer B.Cu) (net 25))
 (segment (start 81.28 94.689913) (end 93.270087 106.68) (width 1.2) (layer B.Cu) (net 25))
 (segment (start 81.28 93.98) (end 81.28 94.689913) (width 1.2) (layer B.Cu) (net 25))
 (segment (start 93.270087 106.68) (end 105.029999 106.68) (width 1.2) (layer B.Cu) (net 25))
 (segment (start 109.22 68.58) (end 109.22 71.12) (width 1.2) (layer B.Cu) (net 16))
 (segment (start 109.22 71.12) (end 111.76 73.66) (width 1.2) (layer B.Cu) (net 16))
 (segment (start 111.76 73.66) (end 111.76 83.439999) (width 1.2) (layer B.Cu) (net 16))
 (segment (start 147.01 66.04) (end 149.86 66.04) (width 1.2) (layer B.Cu) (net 29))
 (segment (start 143.53 62.56) (end 147.01 66.04) (width 1.2) (layer B.Cu) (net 29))
 (segment (start 121.92 60.96) (end 127 60.96) (width 1.2) (layer B.Cu) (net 1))
 (via (at 109.22 76.2) (size 0.8) (drill 0.4) (layers F.Cu B.Cu) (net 1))
 (segment (start 106.68 76.2) (end 109.22 76.2) (width 1.2) (layer B.Cu) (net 1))
 (segment (start 134.62 73.66) (end 134.62 76.2) (width 1.2) (layer B.Cu) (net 1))
 (segment (start 134.62 76.2) (end 134.62 76.2) (width 1.2) (layer B.Cu) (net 1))
 (via (at 134.62 76.2) (size 0.8) (drill 0.4) (layers F.Cu B.Cu) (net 1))
 (segment (start 109.22 76.2) (end 134.62 76.2) (width 1.2) (layer F.Cu) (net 1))
 (segment (start 128.42 60.96) (end 134.62 67.16) (width 1.2) (layer B.Cu) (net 1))
 (segment (start 127 60.96) (end 128.42 60.96) (width 1.2) (layer B.Cu) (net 1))
 (segment (start 134.62 67.16) (end 134.62 73.66) (width 1.2) (layer B.Cu) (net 1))
 (segment (start 114.3 60.96) (end 114.3 58.42) (width 1.2) (layer B.Cu) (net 7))
 (segment (start 114.3 58.42) (end 116.84 55.88) (width 1.2) (layer B.Cu) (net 7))
 (segment (start 127 55.88) (end 116.84 55.88) (width 1.2) (layer B.Cu) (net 7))
 (segment (start 111.76 58.42) (end 116.84 53.34) (width 1.2) (layer B.Cu) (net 9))
 (segment (start 111.76 60.96) (end 111.76 58.42) (width 1.2) (layer B.Cu) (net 9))
 (segment (start 127 53.34) (end 116.84 53.34) (width 1.2) (layer B.Cu) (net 9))
 (segment (start 83.82 63.5) (end 83.82 92.71) (width 1.2) (layer B.Cu) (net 23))
 (segment (start 91.44 60.96) (end 91.44 63.5) (width 1.2) (layer B.Cu) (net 23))
 (segment (start 91.44 63.5) (end 83.82 63.5) (width 1.2) (layer B.Cu) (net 23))
 (segment (start 83.82 92.71) (end 95.25 104.14) (width 1.2) (layer B.Cu) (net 23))
 (segment (start 95.25 104.14) (end 105.029999 104.14) (width 1.2) (layer B.Cu) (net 23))
 (segment (start 86.36 66.04) (end 86.36 90.17) (width 1.2) (layer B.Cu) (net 21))
 (segment (start 93.98 60.96) (end 93.98 66.04) (width 1.2) (layer B.Cu) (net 21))
 (segment (start 93.98 66.04) (end 86.36 66.04) (width 1.2) (layer B.Cu) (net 21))
 (segment (start 86.36 90.17) (end 86.36 91.44) (width 1.2) (layer B.Cu) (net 21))
 (segment (start 86.36 91.44) (end 96.52 101.6) (width 1.2) (layer B.Cu) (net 21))
 (segment (start 96.52 101.6) (end 105.029999 101.6) (width 1.2) (layer B.Cu) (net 21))
 (segment (start 83.82 58.42) (end 83.82 55.88) (width 1.2) (layer B.Cu) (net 19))
 (segment (start 96.52 58.42) (end 83.82 58.42) (width 1.2) (layer B.Cu) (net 19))
 (segment (start 78.74 58.42) (end 76.2 58.42) (width 1.2) (layer B.Cu) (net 19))
 (segment (start 76.2 55.88) (end 77.32 55.88) (width 1.2) (layer B.Cu) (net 19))
 (segment (start 83.82 58.42) (end 78.74 58.42) (width 1.2) (layer B.Cu) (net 19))
 (segment (start 96.52 60.96) (end 96.52 58.42) (width 1.2) (layer B.Cu) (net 19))
 (segment (start 76.2 58.42) (end 76.2 55.88) (width 1.2) (layer B.Cu) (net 19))
 (segment (start 78.74 58.42) (end 78.74 95.25) (width 1.2) (layer B.Cu) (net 19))
 (segment (start 78.74 95.25) (end 92.71 109.22) (width 1.2) (layer B.Cu) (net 19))
 (segment (start 92.71 109.22) (end 105.029999 109.22) (width 1.2) (layer B.Cu) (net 19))
 (segment (start 109.22 66.04) (end 124.46 66.04) (width 1.2) (layer B.Cu) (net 11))
 (segment (start 109.22 60.96) (end 109.22 66.04) (width 1.2) (layer B.Cu) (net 11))
 (segment (start 124.46 66.04) (end 124.46 71.12) (width 1.2) (layer B.Cu) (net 11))
 (segment (start 124.46 71.12) (end 127 73.66) (width 1.2) (layer B.Cu) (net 11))
 (segment (start 127 73.66) (end 127 83.439999) (width 1.2) (layer B.Cu) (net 11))
 (segment (start 88.9 68.58) (end 88.9 90.17) (width 1.2) (layer B.Cu) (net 2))
 (segment (start 88.9 90.17) (end 88.9 91.44) (width 1.2) (layer B.Cu) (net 2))
 (segment (start 88.9 91.44) (end 96.52 99.06) (width 1.2) (layer B.Cu) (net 2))
 (segment (start 96.52 99.06) (end 105.029999 99.06) (width 1.2) (layer B.Cu) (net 2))
 (segment (start 91.44 68.58) (end 91.44 90.17) (width 1.2) (layer B.Cu) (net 4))
 (segment (start 91.44 90.17) (end 97.79 96.52) (width 1.2) (layer B.Cu) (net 4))
 (segment (start 97.79 96.52) (end 105.029999 96.52) (width 1.2) (layer B.Cu) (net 4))
 (segment (start 111.76 71.12) (end 111.76 68.58) (width 1.2) (layer B.Cu) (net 18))
 (segment (start 114.3 73.66) (end 111.76 71.12) (width 1.2) (layer B.Cu) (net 18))
 (segment (start 114.3 73.66) (end 114.3 83.439999) (width 1.2) (layer B.Cu) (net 18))
 (segment (start 114.3 71.12) (end 114.3 68.58) (width 1.2) (layer B.Cu) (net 20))
 (segment (start 116.84 73.66) (end 114.3 71.12) (width 1.2) (layer B.Cu) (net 20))
 (segment (start 116.84 73.66) (end 116.84 83.439999) (width 1.2) (layer B.Cu) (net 20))
 (segment (start 116.84 68.58) (end 116.84 71.12) (width 1.2) (layer B.Cu) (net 22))
 (segment (start 116.84 71.12) (end 119.38 73.66) (width 1.2) (layer B.Cu) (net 22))
 (segment (start 119.38 73.66) (end 119.38 83.439999) (width 1.2) (layer B.Cu) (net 22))
 (segment (start 121.92 68.58) (end 121.92 71.12) (width 1.2) (layer B.Cu) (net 26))
 (segment (start 121.92 71.12) (end 124.46 73.66) (width 1.2) (layer B.Cu) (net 26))
 (segment (start 124.46 73.66) (end 124.46 83.439999) (width 1.2) (layer B.Cu) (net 26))
 (segment (start 116.84 63.5) (end 124.46 63.5) (width 1.2) (layer B.Cu) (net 5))
 (segment (start 116.84 60.96) (end 116.84 63.5) (width 1.2) (layer B.Cu) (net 5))
 (segment (start 124.46 63.5) (end 127 66.04) (width 1.2) (layer B.Cu) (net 5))
 (segment (start 127 66.04) (end 127 71.12) (width 1.2) (layer B.Cu) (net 5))
 (segment (start 127 71.244002) (end 129.54 73.66) (width 1.2) (layer B.Cu) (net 5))
 (segment (start 129.54 73.66) (end 129.54 83.439999) (width 1.2) (layer B.Cu) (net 5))
 (segment (start 137.16 66.04) (end 137.16 76.2) (width 1.2) (layer B.Cu) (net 3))
 (segment (start 129.54 58.42) (end 137.16 66.04) (width 1.2) (layer B.Cu) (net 3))
 (segment (start 119.38 60.96) (end 119.38 58.42) (width 1.2) (layer B.Cu) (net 3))
 (segment (start 119.38 58.42) (end 129.54 58.42) (width 1.2) (layer B.Cu) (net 3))
 (segment (start 132.08 81.28) (end 132.08 83.439999) (width 1.2) (layer B.Cu) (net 3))
 (segment (start 137.16 76.2) (end 132.08 81.28) (width 1.2) (layer B.Cu) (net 3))
 (segment (start 119.38 71.12) (end 119.38 68.58) (width 1.2) (layer B.Cu) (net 24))
 (segment (start 121.92 73.66) (end 119.38 71.12) (width 1.2) (layer B.Cu) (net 24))
 (segment (start 121.92 73.66) (end 121.92 83.439999) (width 1.2) (layer B.Cu) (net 24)))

